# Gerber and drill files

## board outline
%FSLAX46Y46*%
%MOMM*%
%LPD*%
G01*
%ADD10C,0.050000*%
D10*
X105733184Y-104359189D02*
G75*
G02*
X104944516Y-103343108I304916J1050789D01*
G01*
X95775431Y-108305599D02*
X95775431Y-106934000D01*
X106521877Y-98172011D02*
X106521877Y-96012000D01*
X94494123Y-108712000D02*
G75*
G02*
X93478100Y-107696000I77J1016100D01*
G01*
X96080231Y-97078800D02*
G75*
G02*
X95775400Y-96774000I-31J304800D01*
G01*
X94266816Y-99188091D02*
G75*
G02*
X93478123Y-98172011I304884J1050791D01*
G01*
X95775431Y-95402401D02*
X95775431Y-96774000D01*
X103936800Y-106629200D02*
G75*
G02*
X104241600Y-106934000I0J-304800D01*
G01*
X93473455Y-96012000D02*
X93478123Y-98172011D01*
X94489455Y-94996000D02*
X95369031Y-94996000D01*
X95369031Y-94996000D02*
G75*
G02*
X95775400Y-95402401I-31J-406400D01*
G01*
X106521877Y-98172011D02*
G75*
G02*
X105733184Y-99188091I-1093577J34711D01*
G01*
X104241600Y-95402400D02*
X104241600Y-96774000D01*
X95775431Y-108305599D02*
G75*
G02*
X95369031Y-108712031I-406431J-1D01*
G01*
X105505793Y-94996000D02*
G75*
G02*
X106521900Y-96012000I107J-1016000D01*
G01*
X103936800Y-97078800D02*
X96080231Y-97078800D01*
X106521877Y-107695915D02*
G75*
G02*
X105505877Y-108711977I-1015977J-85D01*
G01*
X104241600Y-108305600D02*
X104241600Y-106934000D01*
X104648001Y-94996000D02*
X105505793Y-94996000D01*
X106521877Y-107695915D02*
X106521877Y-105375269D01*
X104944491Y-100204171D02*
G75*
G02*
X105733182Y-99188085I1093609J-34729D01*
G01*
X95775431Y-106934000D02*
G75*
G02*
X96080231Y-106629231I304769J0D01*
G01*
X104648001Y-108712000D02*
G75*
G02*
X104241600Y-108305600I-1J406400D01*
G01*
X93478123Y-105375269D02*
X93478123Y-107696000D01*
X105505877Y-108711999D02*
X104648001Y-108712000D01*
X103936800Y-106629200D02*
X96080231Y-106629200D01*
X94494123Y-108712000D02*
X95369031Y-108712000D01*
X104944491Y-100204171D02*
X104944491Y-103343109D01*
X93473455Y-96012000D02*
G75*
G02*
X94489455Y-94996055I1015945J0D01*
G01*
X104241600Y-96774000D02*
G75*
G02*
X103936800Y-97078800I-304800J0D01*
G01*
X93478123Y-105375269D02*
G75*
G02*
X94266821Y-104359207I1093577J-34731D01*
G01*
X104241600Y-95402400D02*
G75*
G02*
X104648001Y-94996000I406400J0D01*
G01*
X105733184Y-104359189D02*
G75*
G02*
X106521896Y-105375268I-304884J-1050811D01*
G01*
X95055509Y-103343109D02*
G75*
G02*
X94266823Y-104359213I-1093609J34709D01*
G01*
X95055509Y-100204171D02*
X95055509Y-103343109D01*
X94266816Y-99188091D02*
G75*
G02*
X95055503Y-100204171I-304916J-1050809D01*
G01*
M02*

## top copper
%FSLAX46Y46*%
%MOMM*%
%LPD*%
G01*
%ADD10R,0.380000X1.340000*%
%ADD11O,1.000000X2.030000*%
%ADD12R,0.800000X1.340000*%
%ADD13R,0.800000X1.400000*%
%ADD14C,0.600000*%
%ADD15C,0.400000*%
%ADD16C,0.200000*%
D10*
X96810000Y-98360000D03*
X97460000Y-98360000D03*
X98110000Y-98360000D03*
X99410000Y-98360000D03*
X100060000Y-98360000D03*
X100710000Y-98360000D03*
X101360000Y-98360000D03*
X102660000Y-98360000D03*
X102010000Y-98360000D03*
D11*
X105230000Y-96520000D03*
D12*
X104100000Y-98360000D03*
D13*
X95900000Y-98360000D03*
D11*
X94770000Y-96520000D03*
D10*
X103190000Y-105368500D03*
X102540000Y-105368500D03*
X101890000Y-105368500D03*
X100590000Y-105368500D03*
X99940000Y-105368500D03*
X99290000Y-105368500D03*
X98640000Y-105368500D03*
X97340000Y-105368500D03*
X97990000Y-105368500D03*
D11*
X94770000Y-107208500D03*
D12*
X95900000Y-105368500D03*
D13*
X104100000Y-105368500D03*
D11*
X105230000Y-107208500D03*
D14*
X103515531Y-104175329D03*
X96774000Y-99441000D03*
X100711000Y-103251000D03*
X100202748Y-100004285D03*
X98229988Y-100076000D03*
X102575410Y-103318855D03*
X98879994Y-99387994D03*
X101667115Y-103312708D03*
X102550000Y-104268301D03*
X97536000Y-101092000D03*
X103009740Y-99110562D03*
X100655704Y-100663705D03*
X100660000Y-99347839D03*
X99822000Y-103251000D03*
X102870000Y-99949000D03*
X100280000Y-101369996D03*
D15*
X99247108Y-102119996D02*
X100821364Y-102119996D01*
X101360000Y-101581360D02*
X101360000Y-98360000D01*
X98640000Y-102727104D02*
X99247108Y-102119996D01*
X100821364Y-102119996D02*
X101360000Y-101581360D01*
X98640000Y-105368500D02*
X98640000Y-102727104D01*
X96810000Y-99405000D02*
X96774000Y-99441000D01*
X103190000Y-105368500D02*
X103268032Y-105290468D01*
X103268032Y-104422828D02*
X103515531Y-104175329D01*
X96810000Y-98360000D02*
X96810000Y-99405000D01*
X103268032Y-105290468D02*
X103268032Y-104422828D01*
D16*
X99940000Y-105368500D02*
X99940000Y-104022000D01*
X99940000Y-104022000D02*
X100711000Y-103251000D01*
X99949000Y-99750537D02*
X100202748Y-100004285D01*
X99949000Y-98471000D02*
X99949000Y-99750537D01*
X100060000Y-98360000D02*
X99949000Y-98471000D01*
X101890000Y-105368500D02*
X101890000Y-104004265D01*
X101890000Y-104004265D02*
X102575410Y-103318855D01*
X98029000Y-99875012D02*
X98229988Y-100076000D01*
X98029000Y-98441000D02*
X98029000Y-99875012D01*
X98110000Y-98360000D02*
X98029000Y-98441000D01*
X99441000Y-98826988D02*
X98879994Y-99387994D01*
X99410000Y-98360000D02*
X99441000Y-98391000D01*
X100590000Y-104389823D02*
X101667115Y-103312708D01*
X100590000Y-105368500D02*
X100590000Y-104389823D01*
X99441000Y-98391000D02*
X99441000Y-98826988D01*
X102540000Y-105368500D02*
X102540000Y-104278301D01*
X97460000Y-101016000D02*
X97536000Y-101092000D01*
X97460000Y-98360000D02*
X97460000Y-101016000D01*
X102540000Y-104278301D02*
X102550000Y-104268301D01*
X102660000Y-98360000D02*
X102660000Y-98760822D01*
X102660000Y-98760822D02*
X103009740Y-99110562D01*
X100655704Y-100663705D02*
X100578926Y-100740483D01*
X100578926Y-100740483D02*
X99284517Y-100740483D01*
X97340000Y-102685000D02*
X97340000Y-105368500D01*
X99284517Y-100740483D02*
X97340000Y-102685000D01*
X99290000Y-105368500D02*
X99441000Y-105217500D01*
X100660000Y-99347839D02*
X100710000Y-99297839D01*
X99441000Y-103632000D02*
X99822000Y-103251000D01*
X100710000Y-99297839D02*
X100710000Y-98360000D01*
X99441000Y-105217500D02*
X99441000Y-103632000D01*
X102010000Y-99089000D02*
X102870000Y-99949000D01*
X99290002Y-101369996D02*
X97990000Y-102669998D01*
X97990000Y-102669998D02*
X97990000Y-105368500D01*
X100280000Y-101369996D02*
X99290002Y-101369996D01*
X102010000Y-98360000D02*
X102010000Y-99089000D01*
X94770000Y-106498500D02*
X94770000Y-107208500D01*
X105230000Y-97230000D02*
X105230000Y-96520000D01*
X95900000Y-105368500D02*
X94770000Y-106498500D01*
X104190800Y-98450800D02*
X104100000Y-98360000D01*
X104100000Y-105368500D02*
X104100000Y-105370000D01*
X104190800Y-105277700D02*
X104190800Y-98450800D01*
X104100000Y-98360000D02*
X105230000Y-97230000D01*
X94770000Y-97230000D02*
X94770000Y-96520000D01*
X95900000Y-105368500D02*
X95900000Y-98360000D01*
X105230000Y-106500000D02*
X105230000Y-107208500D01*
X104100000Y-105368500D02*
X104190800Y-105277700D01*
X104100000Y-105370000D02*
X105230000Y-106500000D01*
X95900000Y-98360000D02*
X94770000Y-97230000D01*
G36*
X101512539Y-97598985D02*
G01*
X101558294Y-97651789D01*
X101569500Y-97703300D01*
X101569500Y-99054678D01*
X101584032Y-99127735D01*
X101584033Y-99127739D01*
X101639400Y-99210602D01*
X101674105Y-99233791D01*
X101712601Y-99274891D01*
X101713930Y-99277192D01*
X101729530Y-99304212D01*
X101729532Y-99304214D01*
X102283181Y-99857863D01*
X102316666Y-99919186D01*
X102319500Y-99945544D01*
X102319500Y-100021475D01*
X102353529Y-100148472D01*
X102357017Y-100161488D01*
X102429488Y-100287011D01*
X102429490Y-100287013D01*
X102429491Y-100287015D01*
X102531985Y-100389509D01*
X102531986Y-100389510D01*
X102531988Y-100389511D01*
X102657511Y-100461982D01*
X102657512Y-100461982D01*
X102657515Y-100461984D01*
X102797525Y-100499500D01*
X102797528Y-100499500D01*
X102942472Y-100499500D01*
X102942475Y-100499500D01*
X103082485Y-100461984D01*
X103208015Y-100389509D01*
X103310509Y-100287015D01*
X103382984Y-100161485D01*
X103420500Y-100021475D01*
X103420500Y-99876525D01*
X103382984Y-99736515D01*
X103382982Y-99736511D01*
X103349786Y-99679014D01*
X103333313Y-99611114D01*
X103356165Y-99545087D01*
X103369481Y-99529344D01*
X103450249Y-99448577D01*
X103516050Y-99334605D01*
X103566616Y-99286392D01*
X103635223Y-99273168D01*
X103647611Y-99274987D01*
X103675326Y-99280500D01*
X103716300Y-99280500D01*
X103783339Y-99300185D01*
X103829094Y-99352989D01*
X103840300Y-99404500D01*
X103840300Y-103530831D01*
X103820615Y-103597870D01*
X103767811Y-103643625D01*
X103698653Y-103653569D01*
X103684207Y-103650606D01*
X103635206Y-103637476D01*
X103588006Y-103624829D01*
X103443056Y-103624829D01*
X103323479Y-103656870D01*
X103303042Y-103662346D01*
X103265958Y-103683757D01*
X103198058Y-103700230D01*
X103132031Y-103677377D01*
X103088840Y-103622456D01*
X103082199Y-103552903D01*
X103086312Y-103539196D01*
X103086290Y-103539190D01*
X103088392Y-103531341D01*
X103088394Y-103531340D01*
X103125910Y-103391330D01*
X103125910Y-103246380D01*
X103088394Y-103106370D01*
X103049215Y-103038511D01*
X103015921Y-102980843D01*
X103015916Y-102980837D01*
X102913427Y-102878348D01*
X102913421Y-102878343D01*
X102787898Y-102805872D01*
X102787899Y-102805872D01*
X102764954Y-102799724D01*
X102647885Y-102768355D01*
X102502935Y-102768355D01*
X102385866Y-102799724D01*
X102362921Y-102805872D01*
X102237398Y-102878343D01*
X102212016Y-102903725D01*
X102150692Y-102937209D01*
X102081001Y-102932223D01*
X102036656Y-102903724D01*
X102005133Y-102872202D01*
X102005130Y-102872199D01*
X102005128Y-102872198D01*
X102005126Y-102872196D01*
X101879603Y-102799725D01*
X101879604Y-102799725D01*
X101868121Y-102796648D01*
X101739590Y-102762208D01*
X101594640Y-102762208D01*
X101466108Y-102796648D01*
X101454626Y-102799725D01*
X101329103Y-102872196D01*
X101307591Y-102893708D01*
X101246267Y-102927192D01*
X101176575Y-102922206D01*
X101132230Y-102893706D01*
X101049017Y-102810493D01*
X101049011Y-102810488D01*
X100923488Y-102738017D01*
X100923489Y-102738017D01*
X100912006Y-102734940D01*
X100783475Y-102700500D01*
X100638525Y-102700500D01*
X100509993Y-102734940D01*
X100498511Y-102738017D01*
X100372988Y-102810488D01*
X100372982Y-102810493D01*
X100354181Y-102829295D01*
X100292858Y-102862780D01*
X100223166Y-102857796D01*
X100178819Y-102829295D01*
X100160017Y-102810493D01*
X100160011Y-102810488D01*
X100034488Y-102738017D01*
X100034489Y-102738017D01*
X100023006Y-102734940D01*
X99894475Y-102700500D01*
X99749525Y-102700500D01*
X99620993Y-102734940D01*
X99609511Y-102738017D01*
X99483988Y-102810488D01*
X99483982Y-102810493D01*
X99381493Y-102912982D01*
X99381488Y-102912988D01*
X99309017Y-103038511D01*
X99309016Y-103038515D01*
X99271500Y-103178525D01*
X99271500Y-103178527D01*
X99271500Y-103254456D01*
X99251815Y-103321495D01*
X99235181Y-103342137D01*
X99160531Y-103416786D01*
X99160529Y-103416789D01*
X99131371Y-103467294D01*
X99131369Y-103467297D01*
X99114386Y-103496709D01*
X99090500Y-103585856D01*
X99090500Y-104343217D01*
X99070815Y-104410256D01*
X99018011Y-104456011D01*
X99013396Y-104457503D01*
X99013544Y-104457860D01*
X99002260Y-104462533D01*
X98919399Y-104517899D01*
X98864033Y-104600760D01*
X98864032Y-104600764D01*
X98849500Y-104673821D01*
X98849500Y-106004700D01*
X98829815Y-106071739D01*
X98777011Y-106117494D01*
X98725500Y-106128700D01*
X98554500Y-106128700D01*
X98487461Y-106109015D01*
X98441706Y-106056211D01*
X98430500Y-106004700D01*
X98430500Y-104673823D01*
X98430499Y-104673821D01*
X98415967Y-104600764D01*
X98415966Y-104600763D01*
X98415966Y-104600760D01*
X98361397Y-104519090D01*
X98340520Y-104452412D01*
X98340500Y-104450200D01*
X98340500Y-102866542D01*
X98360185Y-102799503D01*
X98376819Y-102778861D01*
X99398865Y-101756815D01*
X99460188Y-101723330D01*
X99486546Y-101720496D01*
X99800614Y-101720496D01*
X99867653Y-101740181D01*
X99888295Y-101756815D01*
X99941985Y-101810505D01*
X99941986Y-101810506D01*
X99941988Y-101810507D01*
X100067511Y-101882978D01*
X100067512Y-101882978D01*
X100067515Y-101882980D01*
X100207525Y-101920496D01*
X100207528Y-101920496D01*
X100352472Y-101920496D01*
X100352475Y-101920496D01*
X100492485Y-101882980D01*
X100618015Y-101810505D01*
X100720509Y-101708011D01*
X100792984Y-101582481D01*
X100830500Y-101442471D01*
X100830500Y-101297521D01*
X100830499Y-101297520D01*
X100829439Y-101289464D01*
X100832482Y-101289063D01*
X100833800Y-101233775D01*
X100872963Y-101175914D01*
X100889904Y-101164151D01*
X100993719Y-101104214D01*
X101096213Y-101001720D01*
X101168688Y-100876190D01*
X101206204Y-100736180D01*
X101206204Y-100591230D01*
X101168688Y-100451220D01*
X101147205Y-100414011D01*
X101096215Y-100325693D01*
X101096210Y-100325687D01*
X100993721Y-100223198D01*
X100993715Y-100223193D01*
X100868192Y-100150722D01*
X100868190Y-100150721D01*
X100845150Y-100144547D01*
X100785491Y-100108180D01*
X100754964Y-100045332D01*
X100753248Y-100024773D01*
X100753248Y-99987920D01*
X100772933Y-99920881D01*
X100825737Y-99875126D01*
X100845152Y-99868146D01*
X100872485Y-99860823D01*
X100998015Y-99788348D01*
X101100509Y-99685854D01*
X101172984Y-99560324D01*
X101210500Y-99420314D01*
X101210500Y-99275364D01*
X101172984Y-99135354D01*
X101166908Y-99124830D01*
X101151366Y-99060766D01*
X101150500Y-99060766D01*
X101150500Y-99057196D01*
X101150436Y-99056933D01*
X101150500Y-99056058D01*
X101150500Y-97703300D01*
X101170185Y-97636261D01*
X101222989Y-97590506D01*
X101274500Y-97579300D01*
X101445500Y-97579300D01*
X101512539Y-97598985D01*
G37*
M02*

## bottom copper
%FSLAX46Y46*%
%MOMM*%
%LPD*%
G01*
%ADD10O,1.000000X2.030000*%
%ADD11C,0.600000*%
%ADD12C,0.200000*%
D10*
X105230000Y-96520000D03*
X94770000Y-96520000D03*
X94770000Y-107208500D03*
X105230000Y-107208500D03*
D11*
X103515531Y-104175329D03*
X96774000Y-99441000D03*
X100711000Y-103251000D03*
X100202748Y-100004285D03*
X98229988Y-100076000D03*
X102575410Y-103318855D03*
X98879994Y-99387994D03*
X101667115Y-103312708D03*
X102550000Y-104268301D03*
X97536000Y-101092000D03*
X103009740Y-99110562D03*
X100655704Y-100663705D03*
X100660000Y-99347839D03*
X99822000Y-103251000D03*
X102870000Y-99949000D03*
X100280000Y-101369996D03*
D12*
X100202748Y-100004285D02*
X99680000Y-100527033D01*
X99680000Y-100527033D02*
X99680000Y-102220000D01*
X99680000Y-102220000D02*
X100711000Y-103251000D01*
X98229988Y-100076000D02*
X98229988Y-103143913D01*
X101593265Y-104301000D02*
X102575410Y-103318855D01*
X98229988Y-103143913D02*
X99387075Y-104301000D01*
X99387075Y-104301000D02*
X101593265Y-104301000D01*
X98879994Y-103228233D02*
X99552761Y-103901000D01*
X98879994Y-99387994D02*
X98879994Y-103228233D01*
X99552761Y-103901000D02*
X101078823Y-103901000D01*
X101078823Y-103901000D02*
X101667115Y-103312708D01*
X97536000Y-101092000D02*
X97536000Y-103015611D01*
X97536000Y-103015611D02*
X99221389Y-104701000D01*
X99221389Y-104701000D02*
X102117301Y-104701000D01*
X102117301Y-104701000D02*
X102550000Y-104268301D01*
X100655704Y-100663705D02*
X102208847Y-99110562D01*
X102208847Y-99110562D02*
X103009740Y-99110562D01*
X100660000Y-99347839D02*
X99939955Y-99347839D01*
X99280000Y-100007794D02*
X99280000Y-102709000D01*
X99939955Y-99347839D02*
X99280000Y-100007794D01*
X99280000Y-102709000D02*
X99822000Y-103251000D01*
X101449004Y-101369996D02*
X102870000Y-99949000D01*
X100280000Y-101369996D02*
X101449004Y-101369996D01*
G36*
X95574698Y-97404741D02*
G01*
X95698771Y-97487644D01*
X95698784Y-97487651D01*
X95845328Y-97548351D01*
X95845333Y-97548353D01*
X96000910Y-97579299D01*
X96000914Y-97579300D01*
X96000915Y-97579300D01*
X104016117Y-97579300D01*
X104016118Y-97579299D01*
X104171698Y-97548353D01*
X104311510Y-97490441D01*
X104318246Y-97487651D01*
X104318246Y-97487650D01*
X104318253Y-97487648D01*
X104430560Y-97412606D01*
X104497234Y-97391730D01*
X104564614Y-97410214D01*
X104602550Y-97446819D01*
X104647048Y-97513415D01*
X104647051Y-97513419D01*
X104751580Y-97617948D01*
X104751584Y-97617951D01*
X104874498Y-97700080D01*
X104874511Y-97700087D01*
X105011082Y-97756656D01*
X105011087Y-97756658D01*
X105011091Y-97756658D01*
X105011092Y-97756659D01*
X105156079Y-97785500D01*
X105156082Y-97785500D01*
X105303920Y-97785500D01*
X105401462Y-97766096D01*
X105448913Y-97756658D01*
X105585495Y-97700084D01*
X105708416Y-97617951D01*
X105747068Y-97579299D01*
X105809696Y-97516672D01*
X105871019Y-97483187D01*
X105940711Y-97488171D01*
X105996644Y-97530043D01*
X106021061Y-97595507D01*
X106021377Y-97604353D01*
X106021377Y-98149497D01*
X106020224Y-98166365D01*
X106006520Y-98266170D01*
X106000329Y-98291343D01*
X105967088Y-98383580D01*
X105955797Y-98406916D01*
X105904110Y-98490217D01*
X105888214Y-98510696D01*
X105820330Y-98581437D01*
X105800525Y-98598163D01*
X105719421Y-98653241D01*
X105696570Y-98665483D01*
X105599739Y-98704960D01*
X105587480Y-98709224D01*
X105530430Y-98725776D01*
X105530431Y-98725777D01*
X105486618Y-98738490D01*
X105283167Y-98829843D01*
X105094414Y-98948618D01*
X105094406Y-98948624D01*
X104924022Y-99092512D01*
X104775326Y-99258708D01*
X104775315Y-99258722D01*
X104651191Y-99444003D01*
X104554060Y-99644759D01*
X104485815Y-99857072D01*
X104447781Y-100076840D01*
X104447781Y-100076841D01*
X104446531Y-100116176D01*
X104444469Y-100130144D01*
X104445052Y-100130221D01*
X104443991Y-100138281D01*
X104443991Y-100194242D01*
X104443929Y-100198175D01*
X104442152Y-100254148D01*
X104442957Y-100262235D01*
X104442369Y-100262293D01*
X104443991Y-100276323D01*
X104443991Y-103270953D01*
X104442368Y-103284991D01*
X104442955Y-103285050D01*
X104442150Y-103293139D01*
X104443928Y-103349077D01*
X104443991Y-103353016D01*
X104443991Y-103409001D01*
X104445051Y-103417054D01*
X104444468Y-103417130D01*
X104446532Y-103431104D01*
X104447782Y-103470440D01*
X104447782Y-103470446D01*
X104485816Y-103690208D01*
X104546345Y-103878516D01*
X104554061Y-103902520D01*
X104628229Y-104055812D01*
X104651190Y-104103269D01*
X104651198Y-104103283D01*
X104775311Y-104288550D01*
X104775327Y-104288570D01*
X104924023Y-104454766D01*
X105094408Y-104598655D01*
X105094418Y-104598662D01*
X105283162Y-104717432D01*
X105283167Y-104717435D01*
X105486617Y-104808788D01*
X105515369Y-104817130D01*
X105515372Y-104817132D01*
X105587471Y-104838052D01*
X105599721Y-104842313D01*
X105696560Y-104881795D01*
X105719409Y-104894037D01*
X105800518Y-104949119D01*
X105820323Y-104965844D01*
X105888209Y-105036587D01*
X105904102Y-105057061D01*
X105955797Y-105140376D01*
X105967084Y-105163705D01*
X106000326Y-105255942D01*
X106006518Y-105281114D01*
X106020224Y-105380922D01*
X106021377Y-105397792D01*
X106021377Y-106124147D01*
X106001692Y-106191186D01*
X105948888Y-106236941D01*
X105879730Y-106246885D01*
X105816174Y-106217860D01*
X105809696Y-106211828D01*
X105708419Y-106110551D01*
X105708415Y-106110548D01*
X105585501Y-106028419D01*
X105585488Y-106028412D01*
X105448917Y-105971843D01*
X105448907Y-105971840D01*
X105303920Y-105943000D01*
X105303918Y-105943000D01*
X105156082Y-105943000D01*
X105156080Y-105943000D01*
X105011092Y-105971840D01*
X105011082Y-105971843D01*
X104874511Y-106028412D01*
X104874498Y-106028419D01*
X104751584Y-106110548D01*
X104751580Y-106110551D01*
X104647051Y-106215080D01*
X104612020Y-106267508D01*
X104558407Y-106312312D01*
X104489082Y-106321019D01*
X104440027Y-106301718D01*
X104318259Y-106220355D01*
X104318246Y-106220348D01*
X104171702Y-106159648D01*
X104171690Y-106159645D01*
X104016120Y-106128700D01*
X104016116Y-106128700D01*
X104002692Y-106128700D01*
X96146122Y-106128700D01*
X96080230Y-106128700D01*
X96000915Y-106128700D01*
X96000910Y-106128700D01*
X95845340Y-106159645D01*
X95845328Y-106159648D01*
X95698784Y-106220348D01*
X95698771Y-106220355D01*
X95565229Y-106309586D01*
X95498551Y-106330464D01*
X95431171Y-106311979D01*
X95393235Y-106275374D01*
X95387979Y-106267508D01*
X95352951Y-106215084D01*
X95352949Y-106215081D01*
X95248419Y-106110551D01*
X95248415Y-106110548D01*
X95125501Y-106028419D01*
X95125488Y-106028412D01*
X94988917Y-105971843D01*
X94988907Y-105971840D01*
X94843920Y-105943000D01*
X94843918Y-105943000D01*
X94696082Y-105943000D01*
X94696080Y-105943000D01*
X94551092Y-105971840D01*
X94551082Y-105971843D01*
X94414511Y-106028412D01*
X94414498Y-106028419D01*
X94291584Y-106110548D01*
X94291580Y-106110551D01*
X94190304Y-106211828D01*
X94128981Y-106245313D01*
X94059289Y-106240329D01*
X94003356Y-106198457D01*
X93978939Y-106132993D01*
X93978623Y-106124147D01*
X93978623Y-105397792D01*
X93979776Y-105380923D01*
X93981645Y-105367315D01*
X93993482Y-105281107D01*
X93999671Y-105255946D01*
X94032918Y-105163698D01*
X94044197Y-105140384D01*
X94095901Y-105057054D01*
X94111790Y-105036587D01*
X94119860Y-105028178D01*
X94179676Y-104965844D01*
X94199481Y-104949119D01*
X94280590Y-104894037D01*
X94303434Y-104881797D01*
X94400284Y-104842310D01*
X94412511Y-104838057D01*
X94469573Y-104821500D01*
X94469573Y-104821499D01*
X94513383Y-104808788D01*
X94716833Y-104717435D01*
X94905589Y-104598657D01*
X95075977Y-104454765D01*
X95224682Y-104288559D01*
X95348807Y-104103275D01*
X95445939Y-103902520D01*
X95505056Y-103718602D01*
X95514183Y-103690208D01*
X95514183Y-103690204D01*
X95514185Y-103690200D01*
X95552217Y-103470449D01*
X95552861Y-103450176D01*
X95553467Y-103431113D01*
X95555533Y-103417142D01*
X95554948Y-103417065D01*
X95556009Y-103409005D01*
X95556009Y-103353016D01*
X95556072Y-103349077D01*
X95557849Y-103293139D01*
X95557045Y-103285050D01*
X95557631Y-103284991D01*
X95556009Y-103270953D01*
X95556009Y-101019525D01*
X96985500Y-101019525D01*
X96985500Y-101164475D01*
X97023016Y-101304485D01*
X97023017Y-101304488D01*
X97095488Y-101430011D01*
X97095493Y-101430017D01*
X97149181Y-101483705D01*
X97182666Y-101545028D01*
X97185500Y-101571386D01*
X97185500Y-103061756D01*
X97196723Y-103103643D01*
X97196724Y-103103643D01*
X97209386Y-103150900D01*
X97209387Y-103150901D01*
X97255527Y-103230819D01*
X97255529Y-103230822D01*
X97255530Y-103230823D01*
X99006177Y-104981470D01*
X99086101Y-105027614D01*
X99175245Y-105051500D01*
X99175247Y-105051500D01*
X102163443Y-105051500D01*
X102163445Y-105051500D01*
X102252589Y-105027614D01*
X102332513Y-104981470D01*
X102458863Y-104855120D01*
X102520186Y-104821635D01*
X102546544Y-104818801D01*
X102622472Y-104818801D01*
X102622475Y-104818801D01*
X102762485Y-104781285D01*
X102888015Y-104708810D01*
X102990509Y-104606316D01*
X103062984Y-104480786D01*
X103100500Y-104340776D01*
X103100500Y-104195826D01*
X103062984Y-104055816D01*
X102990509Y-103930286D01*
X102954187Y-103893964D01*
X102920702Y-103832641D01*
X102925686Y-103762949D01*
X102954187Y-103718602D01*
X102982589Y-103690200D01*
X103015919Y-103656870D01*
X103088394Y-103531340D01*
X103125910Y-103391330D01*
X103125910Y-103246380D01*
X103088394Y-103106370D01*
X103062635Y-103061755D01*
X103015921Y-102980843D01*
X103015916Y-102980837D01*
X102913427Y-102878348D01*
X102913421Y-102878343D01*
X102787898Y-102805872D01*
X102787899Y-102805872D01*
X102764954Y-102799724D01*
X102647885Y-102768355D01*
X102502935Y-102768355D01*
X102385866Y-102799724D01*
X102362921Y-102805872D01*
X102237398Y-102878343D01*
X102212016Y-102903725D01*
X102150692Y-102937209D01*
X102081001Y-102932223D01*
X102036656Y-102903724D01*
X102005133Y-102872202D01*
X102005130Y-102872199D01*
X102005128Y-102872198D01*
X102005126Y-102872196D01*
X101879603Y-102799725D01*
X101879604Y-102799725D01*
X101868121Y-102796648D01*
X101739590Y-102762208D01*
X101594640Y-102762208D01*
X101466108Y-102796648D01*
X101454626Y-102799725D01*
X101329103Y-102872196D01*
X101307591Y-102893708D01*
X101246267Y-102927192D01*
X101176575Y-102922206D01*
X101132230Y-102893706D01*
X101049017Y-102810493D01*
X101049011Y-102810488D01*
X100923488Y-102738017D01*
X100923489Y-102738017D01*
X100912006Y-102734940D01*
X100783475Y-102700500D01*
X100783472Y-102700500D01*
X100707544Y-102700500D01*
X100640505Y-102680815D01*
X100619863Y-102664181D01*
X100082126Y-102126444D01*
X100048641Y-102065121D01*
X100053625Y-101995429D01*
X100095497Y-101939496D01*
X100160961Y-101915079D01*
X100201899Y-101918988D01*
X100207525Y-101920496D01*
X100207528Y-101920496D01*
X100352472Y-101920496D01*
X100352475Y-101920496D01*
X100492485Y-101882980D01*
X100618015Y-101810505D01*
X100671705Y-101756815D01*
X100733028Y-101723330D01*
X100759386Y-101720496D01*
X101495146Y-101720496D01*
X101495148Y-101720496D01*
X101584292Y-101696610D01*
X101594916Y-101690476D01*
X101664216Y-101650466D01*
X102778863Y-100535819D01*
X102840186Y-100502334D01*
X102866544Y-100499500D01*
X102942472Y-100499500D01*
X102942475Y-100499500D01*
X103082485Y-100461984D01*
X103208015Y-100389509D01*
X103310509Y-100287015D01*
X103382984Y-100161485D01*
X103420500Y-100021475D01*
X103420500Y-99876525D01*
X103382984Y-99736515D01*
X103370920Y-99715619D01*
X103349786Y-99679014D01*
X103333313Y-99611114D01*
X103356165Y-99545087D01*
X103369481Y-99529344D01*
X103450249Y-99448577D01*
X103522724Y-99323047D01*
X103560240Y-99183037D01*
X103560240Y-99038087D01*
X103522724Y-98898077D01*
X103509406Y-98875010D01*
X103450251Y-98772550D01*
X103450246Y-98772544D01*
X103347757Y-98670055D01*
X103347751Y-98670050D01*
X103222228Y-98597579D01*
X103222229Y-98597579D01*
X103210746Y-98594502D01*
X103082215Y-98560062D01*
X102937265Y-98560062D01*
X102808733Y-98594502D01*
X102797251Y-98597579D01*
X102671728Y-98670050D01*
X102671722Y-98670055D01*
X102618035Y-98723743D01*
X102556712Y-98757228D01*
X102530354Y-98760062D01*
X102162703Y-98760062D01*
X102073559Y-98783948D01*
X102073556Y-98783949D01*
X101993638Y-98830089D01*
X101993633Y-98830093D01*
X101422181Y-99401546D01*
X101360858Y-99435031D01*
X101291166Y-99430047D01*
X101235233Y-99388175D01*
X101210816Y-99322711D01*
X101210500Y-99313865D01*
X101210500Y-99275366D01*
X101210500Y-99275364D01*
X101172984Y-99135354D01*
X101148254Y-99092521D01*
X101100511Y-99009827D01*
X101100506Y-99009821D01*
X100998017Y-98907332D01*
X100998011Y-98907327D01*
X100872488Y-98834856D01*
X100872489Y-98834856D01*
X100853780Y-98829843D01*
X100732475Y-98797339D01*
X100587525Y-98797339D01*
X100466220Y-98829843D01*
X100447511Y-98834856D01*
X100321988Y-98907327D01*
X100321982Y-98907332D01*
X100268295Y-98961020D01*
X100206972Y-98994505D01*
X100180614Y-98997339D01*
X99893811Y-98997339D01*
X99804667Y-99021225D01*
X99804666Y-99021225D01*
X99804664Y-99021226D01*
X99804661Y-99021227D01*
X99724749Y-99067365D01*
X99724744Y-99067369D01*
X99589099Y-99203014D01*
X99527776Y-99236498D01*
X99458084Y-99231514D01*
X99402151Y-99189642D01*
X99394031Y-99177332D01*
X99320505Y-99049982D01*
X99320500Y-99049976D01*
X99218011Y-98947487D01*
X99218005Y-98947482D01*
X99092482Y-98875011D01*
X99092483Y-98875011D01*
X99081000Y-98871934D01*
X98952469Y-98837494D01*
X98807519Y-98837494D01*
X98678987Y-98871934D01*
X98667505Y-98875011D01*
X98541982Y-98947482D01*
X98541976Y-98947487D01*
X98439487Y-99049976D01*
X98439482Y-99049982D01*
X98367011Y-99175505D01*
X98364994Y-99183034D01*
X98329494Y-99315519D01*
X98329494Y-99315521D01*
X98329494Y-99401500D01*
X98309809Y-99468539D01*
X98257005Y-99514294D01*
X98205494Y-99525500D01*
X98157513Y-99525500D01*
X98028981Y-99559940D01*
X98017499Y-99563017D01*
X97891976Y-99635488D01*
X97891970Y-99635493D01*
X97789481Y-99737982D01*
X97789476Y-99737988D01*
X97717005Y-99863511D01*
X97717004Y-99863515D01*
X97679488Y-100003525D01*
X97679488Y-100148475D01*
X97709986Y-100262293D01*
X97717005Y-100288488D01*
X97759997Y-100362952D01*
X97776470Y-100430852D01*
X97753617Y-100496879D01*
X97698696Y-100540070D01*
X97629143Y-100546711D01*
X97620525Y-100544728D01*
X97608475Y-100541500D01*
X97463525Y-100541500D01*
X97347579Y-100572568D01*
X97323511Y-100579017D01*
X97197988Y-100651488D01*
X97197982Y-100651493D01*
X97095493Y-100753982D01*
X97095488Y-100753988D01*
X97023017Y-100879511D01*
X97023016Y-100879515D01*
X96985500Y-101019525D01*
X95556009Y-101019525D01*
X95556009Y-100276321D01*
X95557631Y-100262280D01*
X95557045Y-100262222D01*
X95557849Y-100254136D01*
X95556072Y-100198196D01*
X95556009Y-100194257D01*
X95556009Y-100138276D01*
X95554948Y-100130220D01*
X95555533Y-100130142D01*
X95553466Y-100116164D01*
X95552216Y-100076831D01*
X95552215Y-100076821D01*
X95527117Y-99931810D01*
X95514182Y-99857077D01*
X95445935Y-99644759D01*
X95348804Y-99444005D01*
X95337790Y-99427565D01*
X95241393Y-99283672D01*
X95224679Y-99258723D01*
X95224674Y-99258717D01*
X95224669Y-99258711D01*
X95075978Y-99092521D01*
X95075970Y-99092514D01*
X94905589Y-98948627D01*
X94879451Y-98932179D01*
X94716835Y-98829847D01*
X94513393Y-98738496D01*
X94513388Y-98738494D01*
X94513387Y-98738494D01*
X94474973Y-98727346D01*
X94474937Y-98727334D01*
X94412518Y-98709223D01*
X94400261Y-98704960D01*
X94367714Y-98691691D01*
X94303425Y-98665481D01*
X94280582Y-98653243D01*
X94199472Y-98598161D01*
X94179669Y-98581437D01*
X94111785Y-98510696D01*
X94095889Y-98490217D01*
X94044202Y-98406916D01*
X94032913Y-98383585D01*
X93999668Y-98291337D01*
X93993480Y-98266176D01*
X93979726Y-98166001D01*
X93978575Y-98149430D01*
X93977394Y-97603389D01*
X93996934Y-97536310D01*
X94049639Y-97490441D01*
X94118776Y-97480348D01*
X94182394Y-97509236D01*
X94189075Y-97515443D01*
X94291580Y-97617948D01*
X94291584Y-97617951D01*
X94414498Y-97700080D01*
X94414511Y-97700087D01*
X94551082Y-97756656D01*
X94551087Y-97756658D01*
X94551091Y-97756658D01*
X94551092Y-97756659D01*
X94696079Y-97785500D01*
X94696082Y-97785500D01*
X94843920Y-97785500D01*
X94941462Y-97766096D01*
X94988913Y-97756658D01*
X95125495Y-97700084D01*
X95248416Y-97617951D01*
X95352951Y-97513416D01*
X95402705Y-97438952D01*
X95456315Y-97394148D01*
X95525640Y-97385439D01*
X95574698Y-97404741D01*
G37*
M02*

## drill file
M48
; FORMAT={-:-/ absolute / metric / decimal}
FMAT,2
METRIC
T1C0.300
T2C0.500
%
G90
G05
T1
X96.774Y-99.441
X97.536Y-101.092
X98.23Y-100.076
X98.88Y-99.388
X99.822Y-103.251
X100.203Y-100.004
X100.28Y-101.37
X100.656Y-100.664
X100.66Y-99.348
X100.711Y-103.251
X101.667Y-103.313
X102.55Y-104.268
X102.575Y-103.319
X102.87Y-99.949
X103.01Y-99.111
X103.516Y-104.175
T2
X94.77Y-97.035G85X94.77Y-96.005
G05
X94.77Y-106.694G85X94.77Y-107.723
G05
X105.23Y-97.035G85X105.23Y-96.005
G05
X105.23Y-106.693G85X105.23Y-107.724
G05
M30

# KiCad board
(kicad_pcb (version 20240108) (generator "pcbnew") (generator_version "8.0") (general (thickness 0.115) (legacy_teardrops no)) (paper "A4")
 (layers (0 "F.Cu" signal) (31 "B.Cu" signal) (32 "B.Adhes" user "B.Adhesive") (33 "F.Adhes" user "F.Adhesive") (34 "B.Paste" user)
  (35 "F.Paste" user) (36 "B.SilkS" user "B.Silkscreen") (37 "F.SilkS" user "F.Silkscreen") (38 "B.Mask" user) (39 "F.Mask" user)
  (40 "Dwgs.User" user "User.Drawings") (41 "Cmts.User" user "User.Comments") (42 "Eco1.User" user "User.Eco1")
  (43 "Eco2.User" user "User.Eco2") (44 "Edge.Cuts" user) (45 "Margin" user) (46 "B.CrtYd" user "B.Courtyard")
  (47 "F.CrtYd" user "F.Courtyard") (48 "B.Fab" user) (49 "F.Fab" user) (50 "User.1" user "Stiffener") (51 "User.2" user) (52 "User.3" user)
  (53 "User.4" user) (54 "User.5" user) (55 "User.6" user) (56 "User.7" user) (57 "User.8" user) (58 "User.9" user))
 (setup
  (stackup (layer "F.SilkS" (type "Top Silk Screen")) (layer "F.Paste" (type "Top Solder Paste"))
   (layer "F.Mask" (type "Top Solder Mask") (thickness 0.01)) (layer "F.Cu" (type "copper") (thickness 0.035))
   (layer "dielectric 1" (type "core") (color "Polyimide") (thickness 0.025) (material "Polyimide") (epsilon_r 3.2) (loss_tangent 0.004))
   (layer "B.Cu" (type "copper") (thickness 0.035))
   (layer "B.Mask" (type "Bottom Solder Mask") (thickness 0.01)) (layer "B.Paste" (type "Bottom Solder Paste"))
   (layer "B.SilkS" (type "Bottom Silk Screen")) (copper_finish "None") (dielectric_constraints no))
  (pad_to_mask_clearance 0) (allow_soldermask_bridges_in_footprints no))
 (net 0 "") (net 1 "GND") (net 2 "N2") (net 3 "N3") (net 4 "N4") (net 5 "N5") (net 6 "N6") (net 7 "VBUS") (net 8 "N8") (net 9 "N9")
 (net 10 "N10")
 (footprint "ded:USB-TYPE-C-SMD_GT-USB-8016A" (layer "F.Cu") (at 100 97.44 180)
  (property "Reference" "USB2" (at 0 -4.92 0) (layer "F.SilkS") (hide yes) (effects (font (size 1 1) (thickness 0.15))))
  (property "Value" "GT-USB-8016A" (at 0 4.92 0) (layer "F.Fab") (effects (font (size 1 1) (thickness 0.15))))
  (pad "A1" smd rect (at 3.19 -0.92 180) (size 0.38 1.34) (layers "F.Cu" "F.Paste" "F.Mask") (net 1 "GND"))
  (pad "A2" smd rect (at 2.54 -0.92 180) (size 0.38 1.34) (layers "F.Cu" "F.Paste" "F.Mask") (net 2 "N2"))
  (pad "A3" smd rect (at 1.89 -0.92 180) (size 0.38 1.34) (layers "F.Cu" "F.Paste" "F.Mask") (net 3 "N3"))
  (pad "A5" smd rect (at 0.59 -0.92 180) (size 0.38 1.34) (layers "F.Cu" "F.Paste" "F.Mask") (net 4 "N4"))
  (pad "A6" smd rect (at -0.06 -0.92 180) (size 0.38 1.34) (layers "F.Cu" "F.Paste" "F.Mask") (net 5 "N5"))
  (pad "A7" smd rect (at -0.71 -0.92 180) (size 0.38 1.34) (layers "F.Cu" "F.Paste" "F.Mask") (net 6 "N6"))
  (pad "A9" smd rect (at -1.36 -0.92 180) (size 0.38 1.34) (layers "F.Cu" "F.Paste" "F.Mask") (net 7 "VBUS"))
  (pad "B10" smd rect (at -2.66 -0.92 180) (size 0.38 1.34) (layers "F.Cu" "F.Paste" "F.Mask") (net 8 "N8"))
  (pad "B11" smd rect (at -2.01 -0.92 180) (size 0.38 1.34) (layers "F.Cu" "F.Paste" "F.Mask") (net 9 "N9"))
  (pad "S1" thru_hole oval (at -5.23 0.92 180) (size 1 2.03) (drill oval 0.500024 1.529994) (layers "*.Cu" "*.Mask")
   (remove_unused_layers no) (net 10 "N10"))
  (pad "S1" smd rect (at -4.1 -0.92 180) (size 0.8 1.34) (layers "F.Cu" "F.Paste" "F.Mask") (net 10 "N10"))
  (pad "S1" smd rect (at 4.1 -0.92 180) (size 0.8 1.4) (layers "F.Cu" "F.Paste" "F.Mask") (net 10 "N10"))
  (pad "S1" thru_hole oval (at 5.23 0.92 180) (size 1 2.03) (drill oval 0.500024 1.530071) (layers "*.Cu" "*.Mask")
   (remove_unused_layers no) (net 10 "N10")))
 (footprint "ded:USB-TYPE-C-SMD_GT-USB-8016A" (layer "F.Cu") (at 100 106.2885)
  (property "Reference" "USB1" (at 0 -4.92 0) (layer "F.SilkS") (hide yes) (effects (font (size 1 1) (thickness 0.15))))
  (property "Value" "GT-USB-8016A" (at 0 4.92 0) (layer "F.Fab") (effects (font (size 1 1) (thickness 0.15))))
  (pad "A1" smd rect (at 3.19 -0.92) (size 0.38 1.34) (layers "F.Cu" "F.Paste" "F.Mask") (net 1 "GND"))
  (pad "A2" smd rect (at 2.54 -0.92) (size 0.38 1.34) (layers "F.Cu" "F.Paste" "F.Mask") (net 2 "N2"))
  (pad "A3" smd rect (at 1.89 -0.92) (size 0.38 1.34) (layers "F.Cu" "F.Paste" "F.Mask") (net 3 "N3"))
  (pad "A5" smd rect (at 0.59 -0.92) (size 0.38 1.34) (layers "F.Cu" "F.Paste" "F.Mask") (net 4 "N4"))
  (pad "A6" smd rect (at -0.06 -0.92) (size 0.38 1.34) (layers "F.Cu" "F.Paste" "F.Mask") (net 5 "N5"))
  (pad "A7" smd rect (at -0.71 -0.92) (size 0.38 1.34) (layers "F.Cu" "F.Paste" "F.Mask") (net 6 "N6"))
  (pad "A9" smd rect (at -1.36 -0.92) (size 0.38 1.34) (layers "F.Cu" "F.Paste" "F.Mask") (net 7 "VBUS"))
  (pad "B10" smd rect (at -2.66 -0.92) (size 0.38 1.34) (layers "F.Cu" "F.Paste" "F.Mask") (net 8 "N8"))
  (pad "B11" smd rect (at -2.01 -0.92) (size 0.38 1.34) (layers "F.Cu" "F.Paste" "F.Mask") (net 9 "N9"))
  (pad "S1" thru_hole oval (at -5.23 0.92) (size 1 2.03) (drill oval 0.500024 1.529994) (layers "*.Cu" "*.Mask") (remove_unused_layers no)
   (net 10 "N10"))
  (pad "S1" smd rect (at -4.1 -0.92) (size 0.8 1.34) (layers "F.Cu" "F.Paste" "F.Mask") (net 10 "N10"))
  (pad "S1" smd rect (at 4.1 -0.92) (size 0.8 1.4) (layers "F.Cu" "F.Paste" "F.Mask") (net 10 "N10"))
  (pad "S1" thru_hole oval (at 5.23 0.92) (size 1 2.03) (drill oval 0.500024 1.530071) (layers "*.Cu" "*.Mask") (remove_unused_layers no)
   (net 10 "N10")))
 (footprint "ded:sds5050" (layer "F.Cu") (at 99.949 101.77364)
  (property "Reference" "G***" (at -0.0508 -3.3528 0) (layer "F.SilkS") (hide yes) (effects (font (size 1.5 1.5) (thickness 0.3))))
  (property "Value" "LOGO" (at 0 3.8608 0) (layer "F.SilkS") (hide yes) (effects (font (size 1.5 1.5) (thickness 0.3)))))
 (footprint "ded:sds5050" (layer "B.Cu") (at 99.9744 101.7524 180)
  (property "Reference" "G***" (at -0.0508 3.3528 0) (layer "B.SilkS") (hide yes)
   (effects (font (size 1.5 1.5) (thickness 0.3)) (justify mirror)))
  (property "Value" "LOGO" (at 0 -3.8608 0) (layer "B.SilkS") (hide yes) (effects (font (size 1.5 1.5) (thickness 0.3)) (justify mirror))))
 (gr_arc (start 105.733184 104.359189) (mid 105.173765 103.97928) (end 104.944491 103.343109) (stroke (width 0.05) (type default))
  (layer "Edge.Cuts"))
 (gr_line (start 95.775431 108.305599) (end 95.775431 106.934) (stroke (width 0.05) (type default)) (layer "Edge.Cuts"))
 (gr_line (start 106.521877 98.172011) (end 106.521877 96.012) (stroke (width 0.05) (type default)) (layer "Edge.Cuts"))
 (gr_arc (start 94.494123 108.712) (mid 93.775703 108.41442) (end 93.478039 107.696) (stroke (width 0.05) (type default))
  (layer "Edge.Cuts"))
 (gr_arc (start 96.080231 97.0788) (mid 95.864705 96.989526) (end 95.775431 96.774) (stroke (width 0.05) (type default)) (layer "Edge.Cuts"))
 (gr_arc (start 94.266816 99.188091) (mid 93.707392 98.808186) (end 93.478123 98.172011) (stroke (width 0.05) (type default))
  (layer "Edge.Cuts"))
 (gr_line (start 95.775431 95.402401) (end 95.775431 96.774) (stroke (width 0.05) (type default)) (layer "Edge.Cuts"))
 (gr_arc (start 103.9368 106.6292) (mid 104.152326 106.718474) (end 104.2416 106.934) (stroke (width 0.05) (type default))
  (layer "Edge.Cuts"))
 (gr_line (start 93.473455 96.012) (end 93.478123 98.172011) (stroke (width 0.05) (type default)) (layer "Edge.Cuts"))
 (gr_line (start 94.489455 94.996) (end 95.369031 94.996) (stroke (width 0.05) (type default)) (layer "Edge.Cuts"))
 (gr_arc (start 95.369031 94.996) (mid 95.6564 95.115032) (end 95.775431 95.402401) (stroke (width 0.05) (type default)) (layer "Edge.Cuts"))
 (gr_arc (start 106.521877 98.172011) (mid 106.292608 98.808186) (end 105.733184 99.188091) (stroke (width 0.05) (type default))
  (layer "Edge.Cuts"))
 (gr_line (start 104.2416 95.4024) (end 104.2416 96.774) (stroke (width 0.05) (type default)) (layer "Edge.Cuts"))
 (gr_arc (start 95.775431 108.305599) (mid 95.6564 108.592968) (end 95.369031 108.712) (stroke (width 0.05) (type default))
  (layer "Edge.Cuts"))
 (gr_arc (start 105.505793 94.996) (mid 106.224283 95.293542) (end 106.521877 96.012) (stroke (width 0.05) (type default))
  (layer "Edge.Cuts"))
 (gr_line (start 103.9368 97.0788) (end 96.080231 97.0788) (stroke (width 0.05) (type default)) (layer "Edge.Cuts"))
 (gr_arc (start 106.521877 107.695915) (mid 106.224328 108.41439) (end 105.505877 108.711999) (stroke (width 0.05) (type default))
  (layer "Edge.Cuts"))
 (gr_line (start 104.2416 108.3056) (end 104.2416 106.934) (stroke (width 0.05) (type default)) (layer "Edge.Cuts"))
 (gr_line (start 104.648001 94.996) (end 105.505793 94.996) (stroke (width 0.05) (type default)) (layer "Edge.Cuts"))
 (gr_line (start 106.521877 107.695915) (end 106.521877 105.375269) (stroke (width 0.05) (type default)) (layer "Edge.Cuts"))
 (gr_arc (start 104.944491 100.204171) (mid 105.173764 99.567998) (end 105.733184 99.188091) (stroke (width 0.05) (type default))
  (layer "Edge.Cuts"))
 (gr_arc (start 95.775431 106.934) (mid 95.864705 106.718474) (end 96.080231 106.6292) (stroke (width 0.05) (type default))
  (layer "Edge.Cuts"))
 (gr_arc (start 104.648001 108.712) (mid 104.360632 108.592969) (end 104.2416 108.3056) (stroke (width 0.05) (type default))
  (layer "Edge.Cuts"))
 (gr_line (start 93.478123 105.375269) (end 93.478123 107.696) (stroke (width 0.05) (type default)) (layer "Edge.Cuts"))
 (gr_line (start 105.505877 108.711999) (end 104.648001 108.712) (stroke (width 0.05) (type default)) (layer "Edge.Cuts"))
 (gr_line (start 103.9368 106.6292) (end 96.080231 106.6292) (stroke (width 0.05) (type default)) (layer "Edge.Cuts"))
 (gr_line (start 94.494123 108.712) (end 95.369031 108.712) (stroke (width 0.05) (type default)) (layer "Edge.Cuts"))
 (gr_line (start 104.944491 100.204171) (end 104.944491 103.343109) (stroke (width 0.05) (type default)) (layer "Edge.Cuts"))
 (gr_arc (start 93.473455 96.012) (mid 93.771032 95.293564) (end 94.489455 94.996) (stroke (width 0.05) (type default)) (layer "Edge.Cuts"))
 (gr_arc (start 104.2416 96.774) (mid 104.152326 96.989526) (end 103.9368 97.0788) (stroke (width 0.05) (type default)) (layer "Edge.Cuts"))
 (gr_arc (start 93.478123 105.375269) (mid 93.707397 104.739098) (end 94.266816 104.359189) (stroke (width 0.05) (type default))
  (layer "Edge.Cuts"))
 (gr_arc (start 104.2416 95.4024) (mid 104.360632 95.115031) (end 104.648001 94.996) (stroke (width 0.05) (type default))
  (layer "Edge.Cuts"))
 (gr_arc (start 105.733184 104.359189) (mid 106.292603 104.739098) (end 106.521877 105.375269) (stroke (width 0.05) (type default))
  (layer "Edge.Cuts"))
 (gr_arc (start 95.055509 103.343109) (mid 94.826235 103.97928) (end 94.266816 104.359189) (stroke (width 0.05) (type default))
  (layer "Edge.Cuts"))
 (gr_line (start 95.055509 100.204171) (end 95.055509 103.343109) (stroke (width 0.05) (type default)) (layer "Edge.Cuts"))
 (gr_arc (start 94.266816 99.188091) (mid 94.826231 99.568001) (end 95.055509 100.204171) (stroke (width 0.05) (type default))
  (layer "Edge.Cuts"))
 (segment (start 99.247108 102.119996) (end 100.821364 102.119996) (width 0.4) (layer "F.Cu") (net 7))
 (segment (start 101.36 101.58136) (end 101.36 98.36) (width 0.4) (layer "F.Cu") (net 7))
 (segment (start 98.64 102.727104) (end 99.247108 102.119996) (width 0.4) (layer "F.Cu") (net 7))
 (segment (start 100.821364 102.119996) (end 101.36 101.58136) (width 0.4) (layer "F.Cu") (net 7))
 (segment (start 98.64 105.3685) (end 98.64 102.727104) (width 0.4) (layer "F.Cu") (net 7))
 (segment (start 96.81 99.405) (end 96.774 99.441) (width 0.4) (layer "F.Cu") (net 1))
 (segment (start 103.19 105.3685) (end 103.268032 105.290468) (width 0.4) (layer "F.Cu") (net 1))
 (segment (start 103.268032 104.422828) (end 103.515531 104.175329) (width 0.4) (layer "F.Cu") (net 1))
 (segment (start 96.81 98.36) (end 96.81 99.405) (width 0.4) (layer "F.Cu") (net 1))
 (segment (start 103.268032 105.290468) (end 103.268032 104.422828) (width 0.4) (layer "F.Cu") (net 1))
 (via (at 103.515531 104.175329) (size 0.6) (drill 0.3) (layers "F.Cu" "B.Cu") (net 1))
 (via (at 96.774 99.441) (size 0.6) (drill 0.3) (layers "F.Cu" "B.Cu") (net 1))
 (segment (start 99.94 105.3685) (end 99.94 104.022) (width 0.2) (layer "F.Cu") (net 5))
 (segment (start 99.94 104.022) (end 100.711 103.251) (width 0.2) (layer "F.Cu") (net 5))
 (segment (start 99.949 99.750537) (end 100.202748 100.004285) (width 0.2) (layer "F.Cu") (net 5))
 (segment (start 99.949 98.471) (end 99.949 99.750537) (width 0.2) (layer "F.Cu") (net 5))
 (segment (start 100.06 98.36) (end 99.949 98.471) (width 0.2) (layer "F.Cu") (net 5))
 (via (at 100.711 103.251) (size 0.6) (drill 0.3) (layers "F.Cu" "B.Cu") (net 5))
 (via (at 100.202748 100.004285) (size 0.6) (drill 0.3) (layers "F.Cu" "B.Cu") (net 5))
 (segment (start 100.202748 100.004285) (end 99.68 100.527033) (width 0.2) (layer "B.Cu") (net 5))
 (segment (start 99.68 100.527033) (end 99.68 102.22) (width 0.2) (layer "B.Cu") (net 5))
 (segment (start 99.68 102.22) (end 100.711 103.251) (width 0.2) (layer "B.Cu") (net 5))
 (segment (start 101.89 105.3685) (end 101.89 104.004265) (width 0.2) (layer "F.Cu") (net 3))
 (segment (start 101.89 104.004265) (end 102.57541 103.318855) (width 0.2) (layer "F.Cu") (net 3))
 (segment (start 98.029 99.875012) (end 98.229988 100.076) (width 0.2) (layer "F.Cu") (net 3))
 (segment (start 98.029 98.441) (end 98.029 99.875012) (width 0.2) (layer "F.Cu") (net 3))
 (segment (start 98.11 98.36) (end 98.029 98.441) (width 0.2) (layer "F.Cu") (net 3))
 (via (at 98.229988 100.076) (size 0.6) (drill 0.3) (layers "F.Cu" "B.Cu") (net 3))
 (via (at 102.57541 103.318855) (size 0.6) (drill 0.3) (layers "F.Cu" "B.Cu") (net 3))
 (segment (start 98.229988 100.076) (end 98.229988 103.143913) (width 0.2) (layer "B.Cu") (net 3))
 (segment (start 101.593265 104.301) (end 102.57541 103.318855) (width 0.2) (layer "B.Cu") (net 3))
 (segment (start 98.229988 103.143913) (end 99.387075 104.301) (width 0.2) (layer "B.Cu") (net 3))
 (segment (start 99.387075 104.301) (end 101.593265 104.301) (width 0.2) (layer "B.Cu") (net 3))
 (segment (start 99.441 98.826988) (end 98.879994 99.387994) (width 0.2) (layer "F.Cu") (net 4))
 (segment (start 99.41 98.36) (end 99.441 98.391) (width 0.2) (layer "F.Cu") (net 4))
 (segment (start 100.59 104.389823) (end 101.667115 103.312708) (width 0.2) (layer "F.Cu") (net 4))
 (segment (start 100.59 105.3685) (end 100.59 104.389823) (width 0.2) (layer "F.Cu") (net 4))
 (segment (start 99.441 98.391) (end 99.441 98.826988) (width 0.2) (layer "F.Cu") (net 4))
 (via (at 98.879994 99.387994) (size 0.6) (drill 0.3) (layers "F.Cu" "B.Cu") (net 4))
 (via (at 101.667115 103.312708) (size 0.6) (drill 0.3) (layers "F.Cu" "B.Cu") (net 4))
 (segment (start 98.879994 103.228233) (end 99.552761 103.901) (width 0.2) (layer "B.Cu") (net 4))
 (segment (start 98.879994 99.387994) (end 98.879994 103.228233) (width 0.2) (layer "B.Cu") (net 4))
 (segment (start 99.552761 103.901) (end 101.078823 103.901) (width 0.2) (layer "B.Cu") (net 4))
 (segment (start 101.078823 103.901) (end 101.667115 103.312708) (width 0.2) (layer "B.Cu") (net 4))
 (segment (start 102.54 105.3685) (end 102.54 104.278301) (width 0.2) (layer "F.Cu") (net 2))
 (segment (start 97.46 101.016) (end 97.536 101.092) (width 0.2) (layer "F.Cu") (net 2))
 (segment (start 97.46 98.36) (end 97.46 101.016) (width 0.2) (layer "F.Cu") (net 2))
 (segment (start 102.54 104.278301) (end 102.55 104.268301) (width 0.2) (layer "F.Cu") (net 2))
 (via (at 102.55 104.268301) (size 0.6) (drill 0.3) (layers "F.Cu" "B.Cu") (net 2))
 (via (at 97.536 101.092) (size 0.6) (drill 0.3) (layers "F.Cu" "B.Cu") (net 2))
 (segment (start 97.536 101.092) (end 97.536 103.015611) (width 0.2) (layer "B.Cu") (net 2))
 (segment (start 97.536 103.015611) (end 99.221389 104.701) (width 0.2) (layer "B.Cu") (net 2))
 (segment (start 99.221389 104.701) (end 102.117301 104.701) (width 0.2) (layer "B.Cu") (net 2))
 (segment (start 102.117301 104.701) (end 102.55 104.268301) (width 0.2) (layer "B.Cu") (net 2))
 (segment (start 102.66 98.36) (end 102.66 98.760822) (width 0.2) (layer "F.Cu") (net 8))
 (segment (start 102.66 98.760822) (end 103.00974 99.110562) (width 0.2) (layer "F.Cu") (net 8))
 (segment (start 100.655704 100.663705) (end 100.578926 100.740483) (width 0.2) (layer "F.Cu") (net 8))
 (segment (start 100.578926 100.740483) (end 99.284517 100.740483) (width 0.2) (layer "F.Cu") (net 8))
 (segment (start 97.34 102.685) (end 97.34 105.3685) (width 0.2) (layer "F.Cu") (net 8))
 (segment (start 99.284517 100.740483) (end 97.34 102.685) (width 0.2) (layer "F.Cu") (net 8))
 (via (at 103.00974 99.110562) (size 0.6) (drill 0.3) (layers "F.Cu" "B.Cu") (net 8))
 (via (at 100.655704 100.663705) (size 0.6) (drill 0.3) (layers "F.Cu" "B.Cu") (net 8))
 (segment (start 100.655704 100.663705) (end 102.208847 99.110562) (width 0.2) (layer "B.Cu") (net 8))
 (segment (start 102.208847 99.110562) (end 103.00974 99.110562) (width 0.2) (layer "B.Cu") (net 8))
 (segment (start 99.29 105.3685) (end 99.441 105.2175) (width 0.2) (layer "F.Cu") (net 6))
 (segment (start 100.66 99.347839) (end 100.71 99.297839) (width 0.2) (layer "F.Cu") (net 6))
 (segment (start 99.441 103.632) (end 99.822 103.251) (width 0.2) (layer "F.Cu") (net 6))
 (segment (start 100.71 99.297839) (end 100.71 98.36) (width 0.2) (layer "F.Cu") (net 6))
 (segment (start 99.441 105.2175) (end 99.441 103.632) (width 0.2) (layer "F.Cu") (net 6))
 (via (at 100.66 99.347839) (size 0.6) (drill 0.3) (layers "F.Cu" "B.Cu") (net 6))
 (via (at 99.822 103.251) (size 0.6) (drill 0.3) (layers "F.Cu" "B.Cu") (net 6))
 (segment (start 100.66 99.347839) (end 99.939955 99.347839) (width 0.2) (layer "B.Cu") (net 6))
 (segment (start 99.28 100.007794) (end 99.28 102.709) (width 0.2) (layer "B.Cu") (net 6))
 (segment (start 99.939955 99.347839) (end 99.28 100.007794) (width 0.2) (layer "B.Cu") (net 6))
 (segment (start 99.28 102.709) (end 99.822 103.251) (width 0.2) (layer "B.Cu") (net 6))
 (segment (start 102.01 99.089) (end 102.87 99.949) (width 0.2) (layer "F.Cu") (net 9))
 (segment (start 99.290002 101.369996) (end 97.99 102.669998) (width 0.2) (layer "F.Cu") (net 9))
 (segment (start 97.99 102.669998) (end 97.99 105.3685) (width 0.2) (layer "F.Cu") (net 9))
 (segment (start 100.28 101.369996) (end 99.290002 101.369996) (width 0.2) (layer "F.Cu") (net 9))
 (segment (start 102.01 98.36) (end 102.01 99.089) (width 0.2) (layer "F.Cu") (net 9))
 (via (at 102.87 99.949) (size 0.6) (drill 0.3) (layers "F.Cu" "B.Cu") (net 9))
 (via (at 100.28 101.369996) (size 0.6) (drill 0.3) (layers "F.Cu" "B.Cu") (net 9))
 (segment (start 101.449004 101.369996) (end 102.87 99.949) (width 0.2) (layer "B.Cu") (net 9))
 (segment (start 100.28 101.369996) (end 101.449004 101.369996) (width 0.2) (layer "B.Cu") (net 9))
 (segment (start 94.77 106.4985) (end 94.77 107.2085) (width 0.2) (layer "F.Cu") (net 10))
 (segment (start 105.23 97.23) (end 105.23 96.52) (width 0.2) (layer "F.Cu") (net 10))
 (segment (start 95.9 105.3685) (end 94.77 106.4985) (width 0.2) (layer "F.Cu") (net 10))
 (segment (start 104.1908 98.4508) (end 104.1 98.36) (width 0.2) (layer "F.Cu") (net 10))
 (segment (start 104.1 105.3685) (end 104.1 105.37) (width 0.2) (layer "F.Cu") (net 10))
 (segment (start 104.1908 105.2777) (end 104.1908 98.4508) (width 0.2) (layer "F.Cu") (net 10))
 (segment (start 104.1 98.36) (end 105.23 97.23) (width 0.2) (layer "F.Cu") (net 10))
 (segment (start 94.77 97.23) (end 94.77 96.52) (width 0.2) (layer "F.Cu") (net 10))
 (segment (start 95.9 105.3685) (end 95.9 98.36) (width 0.2) (layer "F.Cu") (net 10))
 (segment (start 105.23 106.5) (end 105.23 107.2085) (width 0.2) (layer "F.Cu") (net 10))
 (segment (start 104.1 105.3685) (end 104.1908 105.2777) (width 0.2) (layer "F.Cu") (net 10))
 (segment (start 104.1 105.37) (end 105.23 106.5) (width 0.2) (layer "F.Cu") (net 10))
 (segment (start 95.9 98.36) (end 94.77 97.23) (width 0.2) (layer "F.Cu") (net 10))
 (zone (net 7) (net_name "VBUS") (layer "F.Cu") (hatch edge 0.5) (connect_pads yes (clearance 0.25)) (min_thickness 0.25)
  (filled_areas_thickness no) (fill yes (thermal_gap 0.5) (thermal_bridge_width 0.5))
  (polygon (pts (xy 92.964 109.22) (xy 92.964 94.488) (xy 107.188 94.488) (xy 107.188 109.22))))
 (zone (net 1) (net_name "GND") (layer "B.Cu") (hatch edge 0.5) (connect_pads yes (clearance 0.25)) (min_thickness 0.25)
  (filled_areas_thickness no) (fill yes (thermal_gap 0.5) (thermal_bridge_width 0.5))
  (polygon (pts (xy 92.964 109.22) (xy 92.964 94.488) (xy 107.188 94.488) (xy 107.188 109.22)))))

